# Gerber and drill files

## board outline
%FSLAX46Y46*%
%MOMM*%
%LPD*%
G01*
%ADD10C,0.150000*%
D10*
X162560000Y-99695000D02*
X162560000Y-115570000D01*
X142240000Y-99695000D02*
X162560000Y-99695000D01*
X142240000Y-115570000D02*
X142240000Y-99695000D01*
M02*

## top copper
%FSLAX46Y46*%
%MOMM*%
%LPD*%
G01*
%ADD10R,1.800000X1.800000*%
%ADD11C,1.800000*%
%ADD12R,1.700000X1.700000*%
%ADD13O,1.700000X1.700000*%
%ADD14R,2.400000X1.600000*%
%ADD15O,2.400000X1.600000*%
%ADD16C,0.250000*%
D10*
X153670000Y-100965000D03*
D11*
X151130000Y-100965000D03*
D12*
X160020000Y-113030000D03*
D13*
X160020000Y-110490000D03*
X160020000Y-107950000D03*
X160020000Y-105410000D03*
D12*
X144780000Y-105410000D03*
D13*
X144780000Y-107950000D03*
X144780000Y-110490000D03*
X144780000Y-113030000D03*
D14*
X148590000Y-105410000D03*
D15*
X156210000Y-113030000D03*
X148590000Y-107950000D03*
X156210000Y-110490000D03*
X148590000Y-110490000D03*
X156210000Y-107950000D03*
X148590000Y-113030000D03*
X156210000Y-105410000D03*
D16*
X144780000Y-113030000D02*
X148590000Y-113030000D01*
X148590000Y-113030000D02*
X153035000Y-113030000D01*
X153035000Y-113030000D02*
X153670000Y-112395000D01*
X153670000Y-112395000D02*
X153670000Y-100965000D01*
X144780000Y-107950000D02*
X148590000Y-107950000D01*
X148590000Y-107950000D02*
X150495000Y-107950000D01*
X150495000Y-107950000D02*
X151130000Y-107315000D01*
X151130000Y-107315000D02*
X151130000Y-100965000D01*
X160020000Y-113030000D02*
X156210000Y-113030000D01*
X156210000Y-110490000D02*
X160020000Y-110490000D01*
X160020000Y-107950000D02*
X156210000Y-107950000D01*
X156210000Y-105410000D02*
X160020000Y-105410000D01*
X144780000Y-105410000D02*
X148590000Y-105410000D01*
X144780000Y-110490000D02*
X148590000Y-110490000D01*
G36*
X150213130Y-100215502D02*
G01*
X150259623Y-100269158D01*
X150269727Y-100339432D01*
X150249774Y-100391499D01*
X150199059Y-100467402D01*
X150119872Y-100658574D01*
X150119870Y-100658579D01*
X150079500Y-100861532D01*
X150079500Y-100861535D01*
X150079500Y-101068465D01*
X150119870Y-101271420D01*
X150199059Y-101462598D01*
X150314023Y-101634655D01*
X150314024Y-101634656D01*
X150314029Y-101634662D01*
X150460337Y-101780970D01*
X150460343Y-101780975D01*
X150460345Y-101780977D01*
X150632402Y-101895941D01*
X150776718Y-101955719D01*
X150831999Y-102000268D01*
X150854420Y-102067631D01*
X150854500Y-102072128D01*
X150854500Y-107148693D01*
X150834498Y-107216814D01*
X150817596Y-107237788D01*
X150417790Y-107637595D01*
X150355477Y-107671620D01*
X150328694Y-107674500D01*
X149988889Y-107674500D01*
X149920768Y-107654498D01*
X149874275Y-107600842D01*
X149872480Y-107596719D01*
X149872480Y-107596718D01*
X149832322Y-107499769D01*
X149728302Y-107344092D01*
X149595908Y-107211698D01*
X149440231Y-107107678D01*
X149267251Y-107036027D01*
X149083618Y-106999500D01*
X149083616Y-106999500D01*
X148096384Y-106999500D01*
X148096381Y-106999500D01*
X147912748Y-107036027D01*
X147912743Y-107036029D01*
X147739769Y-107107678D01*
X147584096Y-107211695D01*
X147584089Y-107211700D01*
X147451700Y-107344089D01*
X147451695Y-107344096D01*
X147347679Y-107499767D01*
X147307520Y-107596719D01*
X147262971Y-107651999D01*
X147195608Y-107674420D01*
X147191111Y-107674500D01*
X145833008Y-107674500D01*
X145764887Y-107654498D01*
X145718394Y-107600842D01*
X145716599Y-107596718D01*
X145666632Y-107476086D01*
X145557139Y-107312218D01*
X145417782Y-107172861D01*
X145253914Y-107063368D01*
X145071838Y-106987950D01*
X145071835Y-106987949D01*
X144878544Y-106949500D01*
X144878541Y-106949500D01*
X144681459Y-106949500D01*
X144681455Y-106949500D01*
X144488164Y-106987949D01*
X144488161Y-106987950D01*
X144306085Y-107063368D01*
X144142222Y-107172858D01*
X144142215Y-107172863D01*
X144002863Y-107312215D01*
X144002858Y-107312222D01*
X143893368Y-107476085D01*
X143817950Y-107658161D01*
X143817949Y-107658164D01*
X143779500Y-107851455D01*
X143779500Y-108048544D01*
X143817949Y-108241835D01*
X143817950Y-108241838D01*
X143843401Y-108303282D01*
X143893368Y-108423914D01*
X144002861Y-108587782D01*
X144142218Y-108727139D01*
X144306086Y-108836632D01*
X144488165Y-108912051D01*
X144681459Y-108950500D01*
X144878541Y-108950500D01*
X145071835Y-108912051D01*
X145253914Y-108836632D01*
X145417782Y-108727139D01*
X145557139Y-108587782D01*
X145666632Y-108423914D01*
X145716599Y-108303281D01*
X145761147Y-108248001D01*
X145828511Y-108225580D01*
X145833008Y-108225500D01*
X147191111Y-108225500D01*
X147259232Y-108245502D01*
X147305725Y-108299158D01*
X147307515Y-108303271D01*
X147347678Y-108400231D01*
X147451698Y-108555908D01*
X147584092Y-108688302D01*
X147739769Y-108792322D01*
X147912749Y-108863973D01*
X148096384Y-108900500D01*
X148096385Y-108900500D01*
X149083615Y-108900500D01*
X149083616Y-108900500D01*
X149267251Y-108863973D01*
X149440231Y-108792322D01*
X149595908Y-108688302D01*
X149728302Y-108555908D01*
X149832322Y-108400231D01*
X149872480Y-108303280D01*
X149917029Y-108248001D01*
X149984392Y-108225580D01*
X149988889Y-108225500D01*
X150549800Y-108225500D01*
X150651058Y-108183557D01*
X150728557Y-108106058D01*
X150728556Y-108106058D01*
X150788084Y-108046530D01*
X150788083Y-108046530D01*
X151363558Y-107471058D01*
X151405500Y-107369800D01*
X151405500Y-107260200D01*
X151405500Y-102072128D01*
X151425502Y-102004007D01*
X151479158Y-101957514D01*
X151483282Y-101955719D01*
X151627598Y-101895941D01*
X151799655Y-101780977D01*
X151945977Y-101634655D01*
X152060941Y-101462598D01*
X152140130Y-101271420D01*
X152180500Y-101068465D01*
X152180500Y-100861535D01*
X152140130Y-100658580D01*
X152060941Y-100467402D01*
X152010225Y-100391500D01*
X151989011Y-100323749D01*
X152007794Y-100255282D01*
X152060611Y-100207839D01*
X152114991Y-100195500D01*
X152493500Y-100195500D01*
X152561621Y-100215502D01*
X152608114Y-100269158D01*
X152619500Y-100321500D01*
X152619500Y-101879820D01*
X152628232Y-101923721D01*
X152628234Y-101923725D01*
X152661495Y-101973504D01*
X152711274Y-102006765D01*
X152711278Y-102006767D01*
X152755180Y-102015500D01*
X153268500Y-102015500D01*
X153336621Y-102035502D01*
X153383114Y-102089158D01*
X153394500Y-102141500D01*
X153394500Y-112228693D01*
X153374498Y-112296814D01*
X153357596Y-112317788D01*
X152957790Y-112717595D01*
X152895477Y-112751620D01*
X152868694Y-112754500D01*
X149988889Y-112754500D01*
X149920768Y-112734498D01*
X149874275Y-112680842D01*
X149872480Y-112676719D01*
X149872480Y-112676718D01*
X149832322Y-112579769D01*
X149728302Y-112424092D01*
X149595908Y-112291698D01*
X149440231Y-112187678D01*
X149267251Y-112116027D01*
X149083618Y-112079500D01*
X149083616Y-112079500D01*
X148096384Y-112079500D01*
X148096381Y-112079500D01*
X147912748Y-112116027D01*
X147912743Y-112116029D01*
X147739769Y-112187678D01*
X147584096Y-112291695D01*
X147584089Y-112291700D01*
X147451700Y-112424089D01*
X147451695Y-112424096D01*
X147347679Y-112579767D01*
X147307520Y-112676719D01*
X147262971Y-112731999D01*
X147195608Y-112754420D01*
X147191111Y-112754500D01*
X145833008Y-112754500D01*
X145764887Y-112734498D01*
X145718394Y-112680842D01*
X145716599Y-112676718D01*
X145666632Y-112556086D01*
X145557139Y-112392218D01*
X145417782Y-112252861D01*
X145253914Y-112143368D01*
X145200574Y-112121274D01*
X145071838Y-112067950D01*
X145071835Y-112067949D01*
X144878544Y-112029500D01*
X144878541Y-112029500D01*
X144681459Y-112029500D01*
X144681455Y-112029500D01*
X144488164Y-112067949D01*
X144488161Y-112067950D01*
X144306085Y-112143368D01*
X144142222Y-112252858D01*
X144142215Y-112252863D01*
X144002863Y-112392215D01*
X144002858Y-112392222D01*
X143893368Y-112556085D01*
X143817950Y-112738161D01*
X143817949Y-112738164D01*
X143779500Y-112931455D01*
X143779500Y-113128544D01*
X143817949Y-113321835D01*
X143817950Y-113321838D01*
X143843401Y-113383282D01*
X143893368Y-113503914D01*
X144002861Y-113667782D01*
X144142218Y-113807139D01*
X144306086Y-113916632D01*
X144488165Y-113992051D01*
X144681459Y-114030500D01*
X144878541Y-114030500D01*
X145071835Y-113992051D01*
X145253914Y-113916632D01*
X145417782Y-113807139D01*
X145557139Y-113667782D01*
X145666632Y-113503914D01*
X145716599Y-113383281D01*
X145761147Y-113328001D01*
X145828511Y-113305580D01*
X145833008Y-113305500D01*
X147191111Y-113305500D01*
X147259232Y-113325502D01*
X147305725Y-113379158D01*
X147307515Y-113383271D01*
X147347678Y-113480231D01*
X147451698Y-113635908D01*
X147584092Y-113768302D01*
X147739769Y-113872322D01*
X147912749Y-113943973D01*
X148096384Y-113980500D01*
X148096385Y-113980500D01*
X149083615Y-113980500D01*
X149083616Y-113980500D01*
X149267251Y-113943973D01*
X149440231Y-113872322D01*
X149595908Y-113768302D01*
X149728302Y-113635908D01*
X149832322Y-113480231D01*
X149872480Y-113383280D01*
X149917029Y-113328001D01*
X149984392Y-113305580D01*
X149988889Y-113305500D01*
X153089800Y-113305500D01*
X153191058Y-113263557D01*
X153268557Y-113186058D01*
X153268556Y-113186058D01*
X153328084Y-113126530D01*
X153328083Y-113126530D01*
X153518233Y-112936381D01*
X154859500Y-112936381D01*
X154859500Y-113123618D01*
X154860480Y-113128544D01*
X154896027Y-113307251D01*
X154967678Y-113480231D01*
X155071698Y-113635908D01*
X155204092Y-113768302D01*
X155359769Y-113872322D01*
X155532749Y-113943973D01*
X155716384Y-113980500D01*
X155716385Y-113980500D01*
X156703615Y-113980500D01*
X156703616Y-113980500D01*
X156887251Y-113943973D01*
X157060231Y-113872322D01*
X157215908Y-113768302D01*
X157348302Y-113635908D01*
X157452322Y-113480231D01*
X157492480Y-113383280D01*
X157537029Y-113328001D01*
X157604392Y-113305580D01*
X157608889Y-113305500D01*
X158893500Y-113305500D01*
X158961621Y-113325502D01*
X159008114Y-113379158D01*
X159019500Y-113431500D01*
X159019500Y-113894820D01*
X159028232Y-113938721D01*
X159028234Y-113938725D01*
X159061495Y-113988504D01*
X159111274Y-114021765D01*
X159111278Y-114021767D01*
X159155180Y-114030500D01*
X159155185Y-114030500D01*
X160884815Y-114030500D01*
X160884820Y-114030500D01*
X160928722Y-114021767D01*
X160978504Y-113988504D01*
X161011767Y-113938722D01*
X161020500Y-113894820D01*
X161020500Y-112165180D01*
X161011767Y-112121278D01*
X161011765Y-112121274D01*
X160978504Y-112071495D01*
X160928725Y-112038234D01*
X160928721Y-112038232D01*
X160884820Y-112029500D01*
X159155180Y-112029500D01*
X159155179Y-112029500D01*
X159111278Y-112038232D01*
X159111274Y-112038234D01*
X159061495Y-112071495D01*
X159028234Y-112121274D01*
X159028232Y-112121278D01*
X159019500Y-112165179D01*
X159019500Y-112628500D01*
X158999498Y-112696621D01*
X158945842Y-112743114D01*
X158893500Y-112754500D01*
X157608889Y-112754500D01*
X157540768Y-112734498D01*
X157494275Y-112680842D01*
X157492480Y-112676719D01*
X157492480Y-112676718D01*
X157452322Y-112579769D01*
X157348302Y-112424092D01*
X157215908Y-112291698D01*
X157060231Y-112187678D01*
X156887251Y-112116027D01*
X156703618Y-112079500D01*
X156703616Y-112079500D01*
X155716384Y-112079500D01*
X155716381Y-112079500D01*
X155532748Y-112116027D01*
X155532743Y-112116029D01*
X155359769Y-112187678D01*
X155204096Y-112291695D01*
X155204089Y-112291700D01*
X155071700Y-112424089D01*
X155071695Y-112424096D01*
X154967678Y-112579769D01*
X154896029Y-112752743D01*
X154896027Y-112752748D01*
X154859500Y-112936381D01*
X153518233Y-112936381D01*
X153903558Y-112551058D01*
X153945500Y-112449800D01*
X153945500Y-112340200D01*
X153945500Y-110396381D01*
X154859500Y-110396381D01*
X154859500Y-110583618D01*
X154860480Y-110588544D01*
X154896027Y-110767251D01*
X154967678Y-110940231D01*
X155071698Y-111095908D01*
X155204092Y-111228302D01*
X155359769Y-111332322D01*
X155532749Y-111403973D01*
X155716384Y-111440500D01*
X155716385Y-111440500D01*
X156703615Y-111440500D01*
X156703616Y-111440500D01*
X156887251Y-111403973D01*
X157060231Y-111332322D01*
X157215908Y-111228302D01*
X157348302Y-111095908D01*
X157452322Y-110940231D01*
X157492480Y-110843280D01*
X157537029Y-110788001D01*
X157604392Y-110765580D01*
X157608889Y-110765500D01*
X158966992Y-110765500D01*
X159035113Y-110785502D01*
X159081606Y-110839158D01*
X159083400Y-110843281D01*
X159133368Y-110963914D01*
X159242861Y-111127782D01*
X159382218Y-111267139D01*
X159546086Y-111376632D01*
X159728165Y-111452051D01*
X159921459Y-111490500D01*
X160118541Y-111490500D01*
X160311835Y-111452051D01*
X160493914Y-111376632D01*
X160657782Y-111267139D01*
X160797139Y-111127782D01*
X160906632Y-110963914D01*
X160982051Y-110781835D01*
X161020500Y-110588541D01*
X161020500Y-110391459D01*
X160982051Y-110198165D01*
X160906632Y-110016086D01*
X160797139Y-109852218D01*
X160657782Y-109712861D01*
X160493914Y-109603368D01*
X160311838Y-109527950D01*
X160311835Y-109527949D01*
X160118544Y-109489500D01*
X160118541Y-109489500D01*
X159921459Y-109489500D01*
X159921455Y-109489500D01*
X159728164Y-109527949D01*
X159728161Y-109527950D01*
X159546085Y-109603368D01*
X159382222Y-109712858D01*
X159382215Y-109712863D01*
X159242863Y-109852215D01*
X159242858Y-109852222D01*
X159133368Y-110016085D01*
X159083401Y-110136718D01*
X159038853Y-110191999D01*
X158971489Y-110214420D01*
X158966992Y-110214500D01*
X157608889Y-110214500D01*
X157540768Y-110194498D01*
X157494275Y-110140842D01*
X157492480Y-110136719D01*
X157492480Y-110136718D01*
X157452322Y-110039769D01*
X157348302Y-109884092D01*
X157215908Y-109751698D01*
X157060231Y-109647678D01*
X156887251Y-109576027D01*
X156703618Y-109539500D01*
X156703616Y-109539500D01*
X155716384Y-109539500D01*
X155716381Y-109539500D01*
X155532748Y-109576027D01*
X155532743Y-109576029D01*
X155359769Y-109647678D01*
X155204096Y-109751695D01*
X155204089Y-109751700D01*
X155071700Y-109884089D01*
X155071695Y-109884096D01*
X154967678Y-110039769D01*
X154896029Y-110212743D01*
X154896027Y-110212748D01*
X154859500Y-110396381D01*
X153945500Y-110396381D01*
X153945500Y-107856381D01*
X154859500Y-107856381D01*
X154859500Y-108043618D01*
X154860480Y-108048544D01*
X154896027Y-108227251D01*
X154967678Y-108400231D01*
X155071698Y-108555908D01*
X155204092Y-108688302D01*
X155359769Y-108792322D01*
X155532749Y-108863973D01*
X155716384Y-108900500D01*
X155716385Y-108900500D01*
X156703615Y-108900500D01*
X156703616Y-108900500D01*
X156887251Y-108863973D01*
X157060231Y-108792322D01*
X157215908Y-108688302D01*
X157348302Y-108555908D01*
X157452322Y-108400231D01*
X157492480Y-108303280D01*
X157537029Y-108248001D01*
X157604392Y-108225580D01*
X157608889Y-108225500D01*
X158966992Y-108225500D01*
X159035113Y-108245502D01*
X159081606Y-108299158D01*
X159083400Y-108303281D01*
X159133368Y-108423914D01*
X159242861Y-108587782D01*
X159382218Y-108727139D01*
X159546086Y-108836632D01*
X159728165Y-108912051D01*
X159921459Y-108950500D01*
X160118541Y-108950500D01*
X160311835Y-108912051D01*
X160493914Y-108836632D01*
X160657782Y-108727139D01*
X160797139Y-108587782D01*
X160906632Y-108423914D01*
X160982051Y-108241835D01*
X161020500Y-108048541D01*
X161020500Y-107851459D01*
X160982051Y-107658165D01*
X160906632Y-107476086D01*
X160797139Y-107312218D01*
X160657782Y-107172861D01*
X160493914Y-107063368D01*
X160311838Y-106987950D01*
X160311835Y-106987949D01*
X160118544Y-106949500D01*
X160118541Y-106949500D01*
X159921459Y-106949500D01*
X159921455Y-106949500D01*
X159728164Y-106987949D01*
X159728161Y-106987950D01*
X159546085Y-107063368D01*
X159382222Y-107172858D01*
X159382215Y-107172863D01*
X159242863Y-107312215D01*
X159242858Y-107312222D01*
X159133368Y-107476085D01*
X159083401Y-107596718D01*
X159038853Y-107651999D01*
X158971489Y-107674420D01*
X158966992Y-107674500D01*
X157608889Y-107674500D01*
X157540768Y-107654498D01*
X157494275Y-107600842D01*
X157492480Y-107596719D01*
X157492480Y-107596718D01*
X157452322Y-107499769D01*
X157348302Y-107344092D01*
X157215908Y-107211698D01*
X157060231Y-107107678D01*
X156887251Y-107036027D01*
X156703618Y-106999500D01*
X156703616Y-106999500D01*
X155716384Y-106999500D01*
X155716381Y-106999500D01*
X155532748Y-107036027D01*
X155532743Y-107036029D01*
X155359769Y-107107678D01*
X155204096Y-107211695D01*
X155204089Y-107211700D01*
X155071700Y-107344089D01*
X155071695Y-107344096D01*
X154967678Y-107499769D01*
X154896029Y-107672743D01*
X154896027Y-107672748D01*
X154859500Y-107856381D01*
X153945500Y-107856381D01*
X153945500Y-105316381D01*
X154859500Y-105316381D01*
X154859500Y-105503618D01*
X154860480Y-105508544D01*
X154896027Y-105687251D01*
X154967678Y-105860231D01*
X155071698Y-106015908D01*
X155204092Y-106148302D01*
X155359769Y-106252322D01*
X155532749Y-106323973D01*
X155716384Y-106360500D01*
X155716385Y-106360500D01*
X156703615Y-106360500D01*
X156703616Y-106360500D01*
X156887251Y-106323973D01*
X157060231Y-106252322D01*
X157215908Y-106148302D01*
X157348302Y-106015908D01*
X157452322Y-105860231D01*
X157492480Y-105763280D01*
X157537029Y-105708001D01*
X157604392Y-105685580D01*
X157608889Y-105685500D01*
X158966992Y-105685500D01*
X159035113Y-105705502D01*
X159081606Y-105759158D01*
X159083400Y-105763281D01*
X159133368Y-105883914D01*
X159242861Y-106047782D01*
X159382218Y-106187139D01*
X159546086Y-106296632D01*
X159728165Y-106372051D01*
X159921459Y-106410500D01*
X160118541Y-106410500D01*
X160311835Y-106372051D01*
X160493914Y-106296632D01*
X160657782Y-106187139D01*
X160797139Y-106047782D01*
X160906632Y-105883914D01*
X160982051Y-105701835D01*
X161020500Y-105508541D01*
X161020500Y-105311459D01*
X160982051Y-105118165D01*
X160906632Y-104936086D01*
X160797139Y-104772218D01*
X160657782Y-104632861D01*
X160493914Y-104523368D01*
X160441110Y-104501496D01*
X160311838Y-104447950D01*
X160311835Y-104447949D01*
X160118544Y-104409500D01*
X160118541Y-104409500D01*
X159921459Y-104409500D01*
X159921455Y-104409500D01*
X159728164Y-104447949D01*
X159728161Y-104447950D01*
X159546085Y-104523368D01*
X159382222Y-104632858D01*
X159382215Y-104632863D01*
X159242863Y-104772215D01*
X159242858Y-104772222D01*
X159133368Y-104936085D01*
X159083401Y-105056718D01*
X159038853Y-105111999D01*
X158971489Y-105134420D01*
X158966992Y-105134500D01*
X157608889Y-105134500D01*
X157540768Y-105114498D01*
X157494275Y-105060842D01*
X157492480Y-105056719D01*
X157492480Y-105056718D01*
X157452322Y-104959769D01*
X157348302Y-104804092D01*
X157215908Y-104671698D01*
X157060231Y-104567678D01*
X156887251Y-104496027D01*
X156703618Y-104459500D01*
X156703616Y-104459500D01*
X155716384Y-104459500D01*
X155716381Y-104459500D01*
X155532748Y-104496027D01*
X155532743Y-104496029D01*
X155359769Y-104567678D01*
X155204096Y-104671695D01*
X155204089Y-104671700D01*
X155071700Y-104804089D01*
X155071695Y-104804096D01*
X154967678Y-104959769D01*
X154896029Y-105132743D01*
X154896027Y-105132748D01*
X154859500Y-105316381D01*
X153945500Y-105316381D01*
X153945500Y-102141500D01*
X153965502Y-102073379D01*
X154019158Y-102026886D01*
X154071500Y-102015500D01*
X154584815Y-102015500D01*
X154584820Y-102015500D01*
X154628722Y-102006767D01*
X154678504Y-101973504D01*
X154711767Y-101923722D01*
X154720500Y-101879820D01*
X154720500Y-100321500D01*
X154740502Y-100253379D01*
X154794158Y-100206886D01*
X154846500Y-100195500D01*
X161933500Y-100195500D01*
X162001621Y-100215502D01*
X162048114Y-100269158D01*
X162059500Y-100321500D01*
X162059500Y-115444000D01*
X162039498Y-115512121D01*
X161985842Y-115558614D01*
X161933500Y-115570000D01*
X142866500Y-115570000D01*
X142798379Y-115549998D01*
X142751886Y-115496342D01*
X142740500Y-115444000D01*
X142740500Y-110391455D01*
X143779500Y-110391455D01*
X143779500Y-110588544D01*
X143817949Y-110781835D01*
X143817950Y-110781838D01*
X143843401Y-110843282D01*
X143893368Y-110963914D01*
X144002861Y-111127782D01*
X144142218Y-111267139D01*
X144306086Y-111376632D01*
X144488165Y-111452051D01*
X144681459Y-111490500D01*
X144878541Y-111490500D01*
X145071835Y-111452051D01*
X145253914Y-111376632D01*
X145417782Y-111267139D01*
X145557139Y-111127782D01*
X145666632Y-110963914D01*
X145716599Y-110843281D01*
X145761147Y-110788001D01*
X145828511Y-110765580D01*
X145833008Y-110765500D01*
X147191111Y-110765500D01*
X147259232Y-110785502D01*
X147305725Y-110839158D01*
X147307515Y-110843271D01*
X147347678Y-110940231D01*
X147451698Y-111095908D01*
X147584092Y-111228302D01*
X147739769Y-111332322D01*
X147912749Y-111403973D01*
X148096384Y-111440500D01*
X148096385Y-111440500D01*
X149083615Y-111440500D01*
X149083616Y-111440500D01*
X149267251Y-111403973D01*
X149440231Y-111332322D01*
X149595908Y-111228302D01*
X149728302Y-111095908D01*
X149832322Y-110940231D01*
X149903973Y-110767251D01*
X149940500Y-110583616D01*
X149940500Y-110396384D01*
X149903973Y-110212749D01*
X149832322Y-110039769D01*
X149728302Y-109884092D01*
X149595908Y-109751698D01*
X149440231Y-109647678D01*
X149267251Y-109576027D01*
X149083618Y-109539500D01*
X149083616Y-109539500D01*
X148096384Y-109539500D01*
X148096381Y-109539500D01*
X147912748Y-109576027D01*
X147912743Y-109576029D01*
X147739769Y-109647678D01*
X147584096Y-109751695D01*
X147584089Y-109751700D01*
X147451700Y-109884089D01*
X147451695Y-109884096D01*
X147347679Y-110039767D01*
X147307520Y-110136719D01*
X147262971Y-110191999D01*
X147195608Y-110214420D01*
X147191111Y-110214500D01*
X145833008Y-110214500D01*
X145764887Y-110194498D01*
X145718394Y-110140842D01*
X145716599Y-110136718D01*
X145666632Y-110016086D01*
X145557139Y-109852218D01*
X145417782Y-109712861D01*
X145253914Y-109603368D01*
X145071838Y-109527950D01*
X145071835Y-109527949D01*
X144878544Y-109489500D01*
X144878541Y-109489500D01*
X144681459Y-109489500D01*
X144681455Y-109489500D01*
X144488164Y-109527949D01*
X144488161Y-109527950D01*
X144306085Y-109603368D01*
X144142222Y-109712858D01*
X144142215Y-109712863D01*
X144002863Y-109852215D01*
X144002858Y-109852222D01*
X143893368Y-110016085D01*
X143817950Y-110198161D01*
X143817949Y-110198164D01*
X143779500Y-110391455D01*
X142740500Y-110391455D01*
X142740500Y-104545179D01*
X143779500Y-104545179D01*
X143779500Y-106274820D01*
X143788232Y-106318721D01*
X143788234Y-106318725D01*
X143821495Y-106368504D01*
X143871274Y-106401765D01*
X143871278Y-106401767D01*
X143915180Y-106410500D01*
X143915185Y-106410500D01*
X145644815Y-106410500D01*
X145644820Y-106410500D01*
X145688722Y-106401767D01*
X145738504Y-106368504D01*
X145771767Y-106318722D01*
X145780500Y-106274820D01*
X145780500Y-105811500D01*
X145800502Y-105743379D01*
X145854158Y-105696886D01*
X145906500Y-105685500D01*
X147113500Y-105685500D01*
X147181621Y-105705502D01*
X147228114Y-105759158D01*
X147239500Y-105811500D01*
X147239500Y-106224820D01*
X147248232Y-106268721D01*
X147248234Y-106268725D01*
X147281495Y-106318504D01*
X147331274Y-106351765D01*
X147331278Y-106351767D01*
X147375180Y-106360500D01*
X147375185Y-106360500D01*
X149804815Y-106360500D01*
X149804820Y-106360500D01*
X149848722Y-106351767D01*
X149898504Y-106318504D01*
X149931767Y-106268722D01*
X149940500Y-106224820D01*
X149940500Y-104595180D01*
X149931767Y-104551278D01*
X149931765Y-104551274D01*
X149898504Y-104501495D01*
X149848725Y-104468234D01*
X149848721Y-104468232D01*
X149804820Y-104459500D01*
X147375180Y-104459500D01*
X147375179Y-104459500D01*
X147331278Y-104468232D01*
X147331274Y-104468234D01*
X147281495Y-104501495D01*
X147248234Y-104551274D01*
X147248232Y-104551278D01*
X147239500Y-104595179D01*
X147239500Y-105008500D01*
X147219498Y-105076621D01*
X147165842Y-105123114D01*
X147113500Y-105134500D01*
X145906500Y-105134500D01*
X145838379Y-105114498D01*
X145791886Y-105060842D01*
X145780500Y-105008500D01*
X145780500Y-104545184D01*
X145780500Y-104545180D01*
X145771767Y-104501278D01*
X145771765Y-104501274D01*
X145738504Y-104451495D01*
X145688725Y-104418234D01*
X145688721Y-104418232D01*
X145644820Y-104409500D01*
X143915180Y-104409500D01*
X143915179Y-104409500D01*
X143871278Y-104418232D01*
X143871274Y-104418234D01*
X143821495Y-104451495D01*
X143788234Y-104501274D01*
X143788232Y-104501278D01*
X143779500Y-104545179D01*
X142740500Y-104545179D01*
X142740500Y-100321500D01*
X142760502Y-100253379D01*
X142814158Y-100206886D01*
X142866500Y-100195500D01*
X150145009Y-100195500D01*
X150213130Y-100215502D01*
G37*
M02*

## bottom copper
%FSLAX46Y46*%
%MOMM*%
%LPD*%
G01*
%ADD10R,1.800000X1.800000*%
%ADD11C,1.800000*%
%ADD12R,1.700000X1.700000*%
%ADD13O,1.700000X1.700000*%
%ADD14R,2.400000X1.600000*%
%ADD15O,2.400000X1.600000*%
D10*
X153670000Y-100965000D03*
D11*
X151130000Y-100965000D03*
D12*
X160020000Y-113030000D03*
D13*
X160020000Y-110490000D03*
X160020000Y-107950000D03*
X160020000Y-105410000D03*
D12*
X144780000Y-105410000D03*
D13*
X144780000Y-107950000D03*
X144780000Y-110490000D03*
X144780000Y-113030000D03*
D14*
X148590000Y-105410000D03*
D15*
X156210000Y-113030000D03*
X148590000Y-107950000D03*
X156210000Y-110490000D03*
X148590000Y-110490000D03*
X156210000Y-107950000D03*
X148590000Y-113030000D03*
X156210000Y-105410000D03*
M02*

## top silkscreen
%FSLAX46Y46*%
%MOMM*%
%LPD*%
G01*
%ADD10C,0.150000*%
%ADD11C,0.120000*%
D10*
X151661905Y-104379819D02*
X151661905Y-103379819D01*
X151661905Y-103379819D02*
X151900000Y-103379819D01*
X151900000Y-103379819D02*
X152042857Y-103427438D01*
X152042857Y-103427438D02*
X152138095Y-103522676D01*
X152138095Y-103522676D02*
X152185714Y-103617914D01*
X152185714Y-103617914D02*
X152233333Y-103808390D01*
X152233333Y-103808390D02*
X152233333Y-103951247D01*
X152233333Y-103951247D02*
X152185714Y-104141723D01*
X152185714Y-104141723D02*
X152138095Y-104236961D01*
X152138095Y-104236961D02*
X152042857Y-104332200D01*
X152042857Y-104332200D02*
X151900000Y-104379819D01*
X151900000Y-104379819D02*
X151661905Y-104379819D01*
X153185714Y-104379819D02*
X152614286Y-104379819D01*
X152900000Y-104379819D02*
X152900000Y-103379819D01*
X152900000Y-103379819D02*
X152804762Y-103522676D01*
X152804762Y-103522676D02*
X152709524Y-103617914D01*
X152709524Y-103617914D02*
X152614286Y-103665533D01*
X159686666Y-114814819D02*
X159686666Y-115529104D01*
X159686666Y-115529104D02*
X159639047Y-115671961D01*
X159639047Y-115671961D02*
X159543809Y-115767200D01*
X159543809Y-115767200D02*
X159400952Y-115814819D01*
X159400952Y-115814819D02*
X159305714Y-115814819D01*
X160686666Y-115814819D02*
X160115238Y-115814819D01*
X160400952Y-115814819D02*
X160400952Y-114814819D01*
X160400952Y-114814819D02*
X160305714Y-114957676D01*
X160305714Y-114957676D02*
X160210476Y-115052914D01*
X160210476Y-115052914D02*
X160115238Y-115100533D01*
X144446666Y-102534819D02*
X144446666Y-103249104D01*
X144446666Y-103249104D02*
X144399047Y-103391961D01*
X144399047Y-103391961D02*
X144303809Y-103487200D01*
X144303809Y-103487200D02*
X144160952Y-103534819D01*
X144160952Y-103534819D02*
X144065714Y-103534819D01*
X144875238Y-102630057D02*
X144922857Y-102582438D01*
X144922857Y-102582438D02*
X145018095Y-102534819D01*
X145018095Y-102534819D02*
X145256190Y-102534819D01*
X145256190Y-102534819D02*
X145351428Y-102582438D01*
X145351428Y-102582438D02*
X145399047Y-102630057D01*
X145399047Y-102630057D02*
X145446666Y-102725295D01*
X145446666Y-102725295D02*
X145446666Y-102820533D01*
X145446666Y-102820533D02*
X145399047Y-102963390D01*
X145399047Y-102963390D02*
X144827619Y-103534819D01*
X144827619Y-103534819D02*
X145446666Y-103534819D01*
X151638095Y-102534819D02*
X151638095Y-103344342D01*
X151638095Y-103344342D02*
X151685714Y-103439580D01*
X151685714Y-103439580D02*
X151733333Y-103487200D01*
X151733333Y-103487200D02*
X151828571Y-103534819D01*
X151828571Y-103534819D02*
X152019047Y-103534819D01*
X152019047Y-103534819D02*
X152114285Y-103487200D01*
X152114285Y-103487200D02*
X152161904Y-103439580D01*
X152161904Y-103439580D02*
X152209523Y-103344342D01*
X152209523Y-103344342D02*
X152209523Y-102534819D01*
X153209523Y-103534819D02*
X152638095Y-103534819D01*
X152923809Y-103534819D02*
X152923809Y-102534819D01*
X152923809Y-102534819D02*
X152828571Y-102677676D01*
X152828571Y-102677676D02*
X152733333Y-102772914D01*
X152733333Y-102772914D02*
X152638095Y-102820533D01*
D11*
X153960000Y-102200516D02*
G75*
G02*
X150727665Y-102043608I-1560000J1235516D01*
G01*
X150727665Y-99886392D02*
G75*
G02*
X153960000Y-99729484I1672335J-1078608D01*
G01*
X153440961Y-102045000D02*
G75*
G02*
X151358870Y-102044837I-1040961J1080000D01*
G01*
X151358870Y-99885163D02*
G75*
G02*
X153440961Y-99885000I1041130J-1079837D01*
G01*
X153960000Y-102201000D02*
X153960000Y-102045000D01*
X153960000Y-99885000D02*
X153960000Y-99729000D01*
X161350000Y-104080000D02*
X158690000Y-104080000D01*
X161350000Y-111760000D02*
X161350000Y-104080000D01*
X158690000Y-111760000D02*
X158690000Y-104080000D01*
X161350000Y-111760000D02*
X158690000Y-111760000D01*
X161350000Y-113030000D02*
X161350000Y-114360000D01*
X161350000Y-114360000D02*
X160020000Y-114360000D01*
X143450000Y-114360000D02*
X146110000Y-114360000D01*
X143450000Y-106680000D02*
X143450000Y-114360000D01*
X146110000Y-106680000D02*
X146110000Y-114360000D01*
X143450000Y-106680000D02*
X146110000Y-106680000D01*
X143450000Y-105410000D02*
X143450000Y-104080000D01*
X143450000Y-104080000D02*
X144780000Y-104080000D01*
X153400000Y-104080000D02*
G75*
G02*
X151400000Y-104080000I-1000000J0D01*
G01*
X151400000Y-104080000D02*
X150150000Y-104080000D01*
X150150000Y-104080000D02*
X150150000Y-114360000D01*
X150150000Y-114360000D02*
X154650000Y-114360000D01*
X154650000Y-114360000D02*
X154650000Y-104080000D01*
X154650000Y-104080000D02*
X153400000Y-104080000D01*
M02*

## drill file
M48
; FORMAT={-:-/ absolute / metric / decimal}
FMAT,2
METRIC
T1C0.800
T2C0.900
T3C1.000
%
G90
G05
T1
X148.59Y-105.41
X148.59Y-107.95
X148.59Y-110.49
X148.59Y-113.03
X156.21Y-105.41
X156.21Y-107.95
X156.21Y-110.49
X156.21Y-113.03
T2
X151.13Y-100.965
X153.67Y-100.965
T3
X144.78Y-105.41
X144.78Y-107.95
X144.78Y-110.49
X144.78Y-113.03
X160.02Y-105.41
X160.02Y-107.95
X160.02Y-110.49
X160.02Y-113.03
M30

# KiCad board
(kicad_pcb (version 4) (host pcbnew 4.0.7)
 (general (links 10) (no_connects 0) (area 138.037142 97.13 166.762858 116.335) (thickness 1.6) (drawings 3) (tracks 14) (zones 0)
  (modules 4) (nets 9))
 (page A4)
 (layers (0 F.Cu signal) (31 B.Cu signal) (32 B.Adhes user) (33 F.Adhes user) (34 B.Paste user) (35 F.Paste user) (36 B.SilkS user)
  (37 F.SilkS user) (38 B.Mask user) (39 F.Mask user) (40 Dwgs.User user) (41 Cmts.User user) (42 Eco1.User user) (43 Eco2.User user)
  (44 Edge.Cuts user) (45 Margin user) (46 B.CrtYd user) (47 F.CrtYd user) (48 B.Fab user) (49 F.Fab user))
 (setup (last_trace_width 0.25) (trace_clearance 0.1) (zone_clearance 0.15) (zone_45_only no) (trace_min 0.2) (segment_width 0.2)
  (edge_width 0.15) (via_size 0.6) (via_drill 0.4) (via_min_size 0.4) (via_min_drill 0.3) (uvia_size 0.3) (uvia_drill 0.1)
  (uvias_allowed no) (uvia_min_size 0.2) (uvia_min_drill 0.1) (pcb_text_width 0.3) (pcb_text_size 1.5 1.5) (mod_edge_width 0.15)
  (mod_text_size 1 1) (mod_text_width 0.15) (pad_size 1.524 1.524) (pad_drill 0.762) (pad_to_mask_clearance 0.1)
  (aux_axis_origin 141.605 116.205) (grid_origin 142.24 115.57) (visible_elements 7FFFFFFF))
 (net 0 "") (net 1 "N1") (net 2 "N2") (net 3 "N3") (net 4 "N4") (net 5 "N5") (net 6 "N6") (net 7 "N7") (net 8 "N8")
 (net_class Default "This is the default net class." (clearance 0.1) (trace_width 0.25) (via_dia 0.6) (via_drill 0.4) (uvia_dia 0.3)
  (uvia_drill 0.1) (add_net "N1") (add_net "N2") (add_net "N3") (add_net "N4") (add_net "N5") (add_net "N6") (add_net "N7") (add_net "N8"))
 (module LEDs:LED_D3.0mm (layer F.Cu) (at 153.67 100.965 180)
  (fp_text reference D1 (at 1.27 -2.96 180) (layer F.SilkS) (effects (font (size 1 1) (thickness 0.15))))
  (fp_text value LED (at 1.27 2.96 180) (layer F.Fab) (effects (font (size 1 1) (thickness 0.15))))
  (fp_arc (start 1.27 0) (end -0.29 -1.235516) (angle 108.8) (layer F.SilkS) (width 0.12))
  (fp_arc (start 1.27 0) (end -0.29 1.235516) (angle -108.8) (layer F.SilkS) (width 0.12))
  (fp_arc (start 1.27 0) (end 0.229039 -1.08) (angle 87.9) (layer F.SilkS) (width 0.12))
  (fp_arc (start 1.27 0) (end 0.229039 1.08) (angle -87.9) (layer F.SilkS) (width 0.12))
  (fp_line (start -0.29 -1.236) (end -0.29 -1.08) (layer F.SilkS) (width 0.12))
  (fp_line (start -0.29 1.08) (end -0.29 1.236) (layer F.SilkS) (width 0.12))
  (pad 1 thru_hole rect (at 0 0 180) (size 1.8 1.8) (drill 0.9) (layers *.Cu *.Mask) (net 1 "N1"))
  (pad 2 thru_hole circle (at 2.54 0 180) (size 1.8 1.8) (drill 0.9) (layers *.Cu *.Mask) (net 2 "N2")))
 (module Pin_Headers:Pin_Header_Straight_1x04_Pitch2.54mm (layer F.Cu) (at 160.02 113.03 180)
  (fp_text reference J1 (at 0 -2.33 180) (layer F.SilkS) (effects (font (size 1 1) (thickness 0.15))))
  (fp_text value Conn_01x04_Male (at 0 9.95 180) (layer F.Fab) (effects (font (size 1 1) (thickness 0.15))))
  (fp_line (start -1.33 8.95) (end 1.33 8.95) (layer F.SilkS) (width 0.12))
  (fp_line (start -1.33 1.27) (end -1.33 8.95) (layer F.SilkS) (width 0.12))
  (fp_line (start 1.33 1.27) (end 1.33 8.95) (layer F.SilkS) (width 0.12))
  (fp_line (start -1.33 1.27) (end 1.33 1.27) (layer F.SilkS) (width 0.12))
  (fp_line (start -1.33 0) (end -1.33 -1.33) (layer F.SilkS) (width 0.12))
  (fp_line (start -1.33 -1.33) (end 0 -1.33) (layer F.SilkS) (width 0.12))
  (pad 1 thru_hole rect (at 0 0 180) (size 1.7 1.7) (drill 1) (layers *.Cu *.Mask) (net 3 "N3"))
  (pad 2 thru_hole oval (at 0 2.54 180) (size 1.7 1.7) (drill 1) (layers *.Cu *.Mask) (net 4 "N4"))
  (pad 3 thru_hole oval (at 0 5.08 180) (size 1.7 1.7) (drill 1) (layers *.Cu *.Mask) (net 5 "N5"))
  (pad 4 thru_hole oval (at 0 7.62 180) (size 1.7 1.7) (drill 1) (layers *.Cu *.Mask) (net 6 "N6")))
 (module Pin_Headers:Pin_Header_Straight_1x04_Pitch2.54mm (layer F.Cu) (at 144.78 105.41)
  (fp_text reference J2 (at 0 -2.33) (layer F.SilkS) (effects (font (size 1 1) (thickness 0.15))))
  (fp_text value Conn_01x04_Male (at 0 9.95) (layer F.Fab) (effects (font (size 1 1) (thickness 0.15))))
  (fp_line (start -1.33 8.95) (end 1.33 8.95) (layer F.SilkS) (width 0.12))
  (fp_line (start -1.33 1.27) (end -1.33 8.95) (layer F.SilkS) (width 0.12))
  (fp_line (start 1.33 1.27) (end 1.33 8.95) (layer F.SilkS) (width 0.12))
  (fp_line (start -1.33 1.27) (end 1.33 1.27) (layer F.SilkS) (width 0.12))
  (fp_line (start -1.33 0) (end -1.33 -1.33) (layer F.SilkS) (width 0.12))
  (fp_line (start -1.33 -1.33) (end 0 -1.33) (layer F.SilkS) (width 0.12))
  (pad 1 thru_hole rect (at 0 0) (size 1.7 1.7) (drill 1) (layers *.Cu *.Mask) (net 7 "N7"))
  (pad 2 thru_hole oval (at 0 2.54) (size 1.7 1.7) (drill 1) (layers *.Cu *.Mask) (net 2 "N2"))
  (pad 3 thru_hole oval (at 0 5.08) (size 1.7 1.7) (drill 1) (layers *.Cu *.Mask) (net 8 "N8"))
  (pad 4 thru_hole oval (at 0 7.62) (size 1.7 1.7) (drill 1) (layers *.Cu *.Mask) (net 1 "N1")))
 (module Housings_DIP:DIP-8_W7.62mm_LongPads (layer F.Cu) (at 148.59 105.41)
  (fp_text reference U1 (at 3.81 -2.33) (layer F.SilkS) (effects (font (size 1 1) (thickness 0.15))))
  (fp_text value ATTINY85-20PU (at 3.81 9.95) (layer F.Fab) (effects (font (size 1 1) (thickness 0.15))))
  (fp_arc (start 3.81 -1.33) (end 2.81 -1.33) (angle -180) (layer F.SilkS) (width 0.12))
  (fp_line (start 2.81 -1.33) (end 1.56 -1.33) (layer F.SilkS) (width 0.12))
  (fp_line (start 1.56 -1.33) (end 1.56 8.95) (layer F.SilkS) (width 0.12))
  (fp_line (start 1.56 8.95) (end 6.06 8.95) (layer F.SilkS) (width 0.12))
  (fp_line (start 6.06 8.95) (end 6.06 -1.33) (layer F.SilkS) (width 0.12))
  (fp_line (start 6.06 -1.33) (end 4.81 -1.33) (layer F.SilkS) (width 0.12))
  (pad 1 thru_hole rect (at 0 0) (size 2.4 1.6) (drill 0.8) (layers *.Cu *.Mask) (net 7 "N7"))
  (pad 5 thru_hole oval (at 7.62 7.62) (size 2.4 1.6) (drill 0.8) (layers *.Cu *.Mask) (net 3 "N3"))
  (pad 2 thru_hole oval (at 0 2.54) (size 2.4 1.6) (drill 0.8) (layers *.Cu *.Mask) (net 2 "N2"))
  (pad 6 thru_hole oval (at 7.62 5.08) (size 2.4 1.6) (drill 0.8) (layers *.Cu *.Mask) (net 4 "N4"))
  (pad 3 thru_hole oval (at 0 5.08) (size 2.4 1.6) (drill 0.8) (layers *.Cu *.Mask) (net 8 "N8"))
  (pad 7 thru_hole oval (at 7.62 2.54) (size 2.4 1.6) (drill 0.8) (layers *.Cu *.Mask) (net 5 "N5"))
  (pad 4 thru_hole oval (at 0 7.62) (size 2.4 1.6) (drill 0.8) (layers *.Cu *.Mask) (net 1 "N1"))
  (pad 8 thru_hole oval (at 7.62 0) (size 2.4 1.6) (drill 0.8) (layers *.Cu *.Mask) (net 6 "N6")))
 (gr_line (start 162.56 99.695) (end 162.56 115.57) (angle 90) (layer Edge.Cuts) (width 0.15))
 (gr_line (start 142.24 99.695) (end 162.56 99.695) (angle 90) (layer Edge.Cuts) (width 0.15))
 (gr_line (start 142.24 115.57) (end 142.24 99.695) (angle 90) (layer Edge.Cuts) (width 0.15))
 (segment (start 144.78 113.03) (end 148.59 113.03) (width 0.25) (layer F.Cu) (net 1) (status C00000))
 (segment (start 148.59 113.03) (end 153.035 113.03) (width 0.25) (layer F.Cu) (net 1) (status 400000))
 (segment (start 153.035 113.03) (end 153.67 112.395) (width 0.25) (layer F.Cu) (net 1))
 (segment (start 153.67 112.395) (end 153.67 100.965) (width 0.25) (layer F.Cu) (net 1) (status 800000))
 (segment (start 144.78 107.95) (end 148.59 107.95) (width 0.25) (layer F.Cu) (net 2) (status C00000))
 (segment (start 148.59 107.95) (end 150.495 107.95) (width 0.25) (layer F.Cu) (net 2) (status 400000))
 (segment (start 150.495 107.95) (end 151.13 107.315) (width 0.25) (layer F.Cu) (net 2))
 (segment (start 151.13 107.315) (end 151.13 100.965) (width 0.25) (layer F.Cu) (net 2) (status 800000))
 (segment (start 160.02 113.03) (end 156.21 113.03) (width 0.25) (layer F.Cu) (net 3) (status C00000))
 (segment (start 156.21 110.49) (end 160.02 110.49) (width 0.25) (layer F.Cu) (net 4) (status C00000))
 (segment (start 160.02 107.95) (end 156.21 107.95) (width 0.25) (layer F.Cu) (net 5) (status C00000))
 (segment (start 156.21 105.41) (end 160.02 105.41) (width 0.25) (layer F.Cu) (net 6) (status C00000))
 (segment (start 144.78 105.41) (end 148.59 105.41) (width 0.25) (layer F.Cu) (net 7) (status C00000))
 (segment (start 144.78 110.49) (end 148.59 110.49) (width 0.25) (layer F.Cu) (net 8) (status C00000))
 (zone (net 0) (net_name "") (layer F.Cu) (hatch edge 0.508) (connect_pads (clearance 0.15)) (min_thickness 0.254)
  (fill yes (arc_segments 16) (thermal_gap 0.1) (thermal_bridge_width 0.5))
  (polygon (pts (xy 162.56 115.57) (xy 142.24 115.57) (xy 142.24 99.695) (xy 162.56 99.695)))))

